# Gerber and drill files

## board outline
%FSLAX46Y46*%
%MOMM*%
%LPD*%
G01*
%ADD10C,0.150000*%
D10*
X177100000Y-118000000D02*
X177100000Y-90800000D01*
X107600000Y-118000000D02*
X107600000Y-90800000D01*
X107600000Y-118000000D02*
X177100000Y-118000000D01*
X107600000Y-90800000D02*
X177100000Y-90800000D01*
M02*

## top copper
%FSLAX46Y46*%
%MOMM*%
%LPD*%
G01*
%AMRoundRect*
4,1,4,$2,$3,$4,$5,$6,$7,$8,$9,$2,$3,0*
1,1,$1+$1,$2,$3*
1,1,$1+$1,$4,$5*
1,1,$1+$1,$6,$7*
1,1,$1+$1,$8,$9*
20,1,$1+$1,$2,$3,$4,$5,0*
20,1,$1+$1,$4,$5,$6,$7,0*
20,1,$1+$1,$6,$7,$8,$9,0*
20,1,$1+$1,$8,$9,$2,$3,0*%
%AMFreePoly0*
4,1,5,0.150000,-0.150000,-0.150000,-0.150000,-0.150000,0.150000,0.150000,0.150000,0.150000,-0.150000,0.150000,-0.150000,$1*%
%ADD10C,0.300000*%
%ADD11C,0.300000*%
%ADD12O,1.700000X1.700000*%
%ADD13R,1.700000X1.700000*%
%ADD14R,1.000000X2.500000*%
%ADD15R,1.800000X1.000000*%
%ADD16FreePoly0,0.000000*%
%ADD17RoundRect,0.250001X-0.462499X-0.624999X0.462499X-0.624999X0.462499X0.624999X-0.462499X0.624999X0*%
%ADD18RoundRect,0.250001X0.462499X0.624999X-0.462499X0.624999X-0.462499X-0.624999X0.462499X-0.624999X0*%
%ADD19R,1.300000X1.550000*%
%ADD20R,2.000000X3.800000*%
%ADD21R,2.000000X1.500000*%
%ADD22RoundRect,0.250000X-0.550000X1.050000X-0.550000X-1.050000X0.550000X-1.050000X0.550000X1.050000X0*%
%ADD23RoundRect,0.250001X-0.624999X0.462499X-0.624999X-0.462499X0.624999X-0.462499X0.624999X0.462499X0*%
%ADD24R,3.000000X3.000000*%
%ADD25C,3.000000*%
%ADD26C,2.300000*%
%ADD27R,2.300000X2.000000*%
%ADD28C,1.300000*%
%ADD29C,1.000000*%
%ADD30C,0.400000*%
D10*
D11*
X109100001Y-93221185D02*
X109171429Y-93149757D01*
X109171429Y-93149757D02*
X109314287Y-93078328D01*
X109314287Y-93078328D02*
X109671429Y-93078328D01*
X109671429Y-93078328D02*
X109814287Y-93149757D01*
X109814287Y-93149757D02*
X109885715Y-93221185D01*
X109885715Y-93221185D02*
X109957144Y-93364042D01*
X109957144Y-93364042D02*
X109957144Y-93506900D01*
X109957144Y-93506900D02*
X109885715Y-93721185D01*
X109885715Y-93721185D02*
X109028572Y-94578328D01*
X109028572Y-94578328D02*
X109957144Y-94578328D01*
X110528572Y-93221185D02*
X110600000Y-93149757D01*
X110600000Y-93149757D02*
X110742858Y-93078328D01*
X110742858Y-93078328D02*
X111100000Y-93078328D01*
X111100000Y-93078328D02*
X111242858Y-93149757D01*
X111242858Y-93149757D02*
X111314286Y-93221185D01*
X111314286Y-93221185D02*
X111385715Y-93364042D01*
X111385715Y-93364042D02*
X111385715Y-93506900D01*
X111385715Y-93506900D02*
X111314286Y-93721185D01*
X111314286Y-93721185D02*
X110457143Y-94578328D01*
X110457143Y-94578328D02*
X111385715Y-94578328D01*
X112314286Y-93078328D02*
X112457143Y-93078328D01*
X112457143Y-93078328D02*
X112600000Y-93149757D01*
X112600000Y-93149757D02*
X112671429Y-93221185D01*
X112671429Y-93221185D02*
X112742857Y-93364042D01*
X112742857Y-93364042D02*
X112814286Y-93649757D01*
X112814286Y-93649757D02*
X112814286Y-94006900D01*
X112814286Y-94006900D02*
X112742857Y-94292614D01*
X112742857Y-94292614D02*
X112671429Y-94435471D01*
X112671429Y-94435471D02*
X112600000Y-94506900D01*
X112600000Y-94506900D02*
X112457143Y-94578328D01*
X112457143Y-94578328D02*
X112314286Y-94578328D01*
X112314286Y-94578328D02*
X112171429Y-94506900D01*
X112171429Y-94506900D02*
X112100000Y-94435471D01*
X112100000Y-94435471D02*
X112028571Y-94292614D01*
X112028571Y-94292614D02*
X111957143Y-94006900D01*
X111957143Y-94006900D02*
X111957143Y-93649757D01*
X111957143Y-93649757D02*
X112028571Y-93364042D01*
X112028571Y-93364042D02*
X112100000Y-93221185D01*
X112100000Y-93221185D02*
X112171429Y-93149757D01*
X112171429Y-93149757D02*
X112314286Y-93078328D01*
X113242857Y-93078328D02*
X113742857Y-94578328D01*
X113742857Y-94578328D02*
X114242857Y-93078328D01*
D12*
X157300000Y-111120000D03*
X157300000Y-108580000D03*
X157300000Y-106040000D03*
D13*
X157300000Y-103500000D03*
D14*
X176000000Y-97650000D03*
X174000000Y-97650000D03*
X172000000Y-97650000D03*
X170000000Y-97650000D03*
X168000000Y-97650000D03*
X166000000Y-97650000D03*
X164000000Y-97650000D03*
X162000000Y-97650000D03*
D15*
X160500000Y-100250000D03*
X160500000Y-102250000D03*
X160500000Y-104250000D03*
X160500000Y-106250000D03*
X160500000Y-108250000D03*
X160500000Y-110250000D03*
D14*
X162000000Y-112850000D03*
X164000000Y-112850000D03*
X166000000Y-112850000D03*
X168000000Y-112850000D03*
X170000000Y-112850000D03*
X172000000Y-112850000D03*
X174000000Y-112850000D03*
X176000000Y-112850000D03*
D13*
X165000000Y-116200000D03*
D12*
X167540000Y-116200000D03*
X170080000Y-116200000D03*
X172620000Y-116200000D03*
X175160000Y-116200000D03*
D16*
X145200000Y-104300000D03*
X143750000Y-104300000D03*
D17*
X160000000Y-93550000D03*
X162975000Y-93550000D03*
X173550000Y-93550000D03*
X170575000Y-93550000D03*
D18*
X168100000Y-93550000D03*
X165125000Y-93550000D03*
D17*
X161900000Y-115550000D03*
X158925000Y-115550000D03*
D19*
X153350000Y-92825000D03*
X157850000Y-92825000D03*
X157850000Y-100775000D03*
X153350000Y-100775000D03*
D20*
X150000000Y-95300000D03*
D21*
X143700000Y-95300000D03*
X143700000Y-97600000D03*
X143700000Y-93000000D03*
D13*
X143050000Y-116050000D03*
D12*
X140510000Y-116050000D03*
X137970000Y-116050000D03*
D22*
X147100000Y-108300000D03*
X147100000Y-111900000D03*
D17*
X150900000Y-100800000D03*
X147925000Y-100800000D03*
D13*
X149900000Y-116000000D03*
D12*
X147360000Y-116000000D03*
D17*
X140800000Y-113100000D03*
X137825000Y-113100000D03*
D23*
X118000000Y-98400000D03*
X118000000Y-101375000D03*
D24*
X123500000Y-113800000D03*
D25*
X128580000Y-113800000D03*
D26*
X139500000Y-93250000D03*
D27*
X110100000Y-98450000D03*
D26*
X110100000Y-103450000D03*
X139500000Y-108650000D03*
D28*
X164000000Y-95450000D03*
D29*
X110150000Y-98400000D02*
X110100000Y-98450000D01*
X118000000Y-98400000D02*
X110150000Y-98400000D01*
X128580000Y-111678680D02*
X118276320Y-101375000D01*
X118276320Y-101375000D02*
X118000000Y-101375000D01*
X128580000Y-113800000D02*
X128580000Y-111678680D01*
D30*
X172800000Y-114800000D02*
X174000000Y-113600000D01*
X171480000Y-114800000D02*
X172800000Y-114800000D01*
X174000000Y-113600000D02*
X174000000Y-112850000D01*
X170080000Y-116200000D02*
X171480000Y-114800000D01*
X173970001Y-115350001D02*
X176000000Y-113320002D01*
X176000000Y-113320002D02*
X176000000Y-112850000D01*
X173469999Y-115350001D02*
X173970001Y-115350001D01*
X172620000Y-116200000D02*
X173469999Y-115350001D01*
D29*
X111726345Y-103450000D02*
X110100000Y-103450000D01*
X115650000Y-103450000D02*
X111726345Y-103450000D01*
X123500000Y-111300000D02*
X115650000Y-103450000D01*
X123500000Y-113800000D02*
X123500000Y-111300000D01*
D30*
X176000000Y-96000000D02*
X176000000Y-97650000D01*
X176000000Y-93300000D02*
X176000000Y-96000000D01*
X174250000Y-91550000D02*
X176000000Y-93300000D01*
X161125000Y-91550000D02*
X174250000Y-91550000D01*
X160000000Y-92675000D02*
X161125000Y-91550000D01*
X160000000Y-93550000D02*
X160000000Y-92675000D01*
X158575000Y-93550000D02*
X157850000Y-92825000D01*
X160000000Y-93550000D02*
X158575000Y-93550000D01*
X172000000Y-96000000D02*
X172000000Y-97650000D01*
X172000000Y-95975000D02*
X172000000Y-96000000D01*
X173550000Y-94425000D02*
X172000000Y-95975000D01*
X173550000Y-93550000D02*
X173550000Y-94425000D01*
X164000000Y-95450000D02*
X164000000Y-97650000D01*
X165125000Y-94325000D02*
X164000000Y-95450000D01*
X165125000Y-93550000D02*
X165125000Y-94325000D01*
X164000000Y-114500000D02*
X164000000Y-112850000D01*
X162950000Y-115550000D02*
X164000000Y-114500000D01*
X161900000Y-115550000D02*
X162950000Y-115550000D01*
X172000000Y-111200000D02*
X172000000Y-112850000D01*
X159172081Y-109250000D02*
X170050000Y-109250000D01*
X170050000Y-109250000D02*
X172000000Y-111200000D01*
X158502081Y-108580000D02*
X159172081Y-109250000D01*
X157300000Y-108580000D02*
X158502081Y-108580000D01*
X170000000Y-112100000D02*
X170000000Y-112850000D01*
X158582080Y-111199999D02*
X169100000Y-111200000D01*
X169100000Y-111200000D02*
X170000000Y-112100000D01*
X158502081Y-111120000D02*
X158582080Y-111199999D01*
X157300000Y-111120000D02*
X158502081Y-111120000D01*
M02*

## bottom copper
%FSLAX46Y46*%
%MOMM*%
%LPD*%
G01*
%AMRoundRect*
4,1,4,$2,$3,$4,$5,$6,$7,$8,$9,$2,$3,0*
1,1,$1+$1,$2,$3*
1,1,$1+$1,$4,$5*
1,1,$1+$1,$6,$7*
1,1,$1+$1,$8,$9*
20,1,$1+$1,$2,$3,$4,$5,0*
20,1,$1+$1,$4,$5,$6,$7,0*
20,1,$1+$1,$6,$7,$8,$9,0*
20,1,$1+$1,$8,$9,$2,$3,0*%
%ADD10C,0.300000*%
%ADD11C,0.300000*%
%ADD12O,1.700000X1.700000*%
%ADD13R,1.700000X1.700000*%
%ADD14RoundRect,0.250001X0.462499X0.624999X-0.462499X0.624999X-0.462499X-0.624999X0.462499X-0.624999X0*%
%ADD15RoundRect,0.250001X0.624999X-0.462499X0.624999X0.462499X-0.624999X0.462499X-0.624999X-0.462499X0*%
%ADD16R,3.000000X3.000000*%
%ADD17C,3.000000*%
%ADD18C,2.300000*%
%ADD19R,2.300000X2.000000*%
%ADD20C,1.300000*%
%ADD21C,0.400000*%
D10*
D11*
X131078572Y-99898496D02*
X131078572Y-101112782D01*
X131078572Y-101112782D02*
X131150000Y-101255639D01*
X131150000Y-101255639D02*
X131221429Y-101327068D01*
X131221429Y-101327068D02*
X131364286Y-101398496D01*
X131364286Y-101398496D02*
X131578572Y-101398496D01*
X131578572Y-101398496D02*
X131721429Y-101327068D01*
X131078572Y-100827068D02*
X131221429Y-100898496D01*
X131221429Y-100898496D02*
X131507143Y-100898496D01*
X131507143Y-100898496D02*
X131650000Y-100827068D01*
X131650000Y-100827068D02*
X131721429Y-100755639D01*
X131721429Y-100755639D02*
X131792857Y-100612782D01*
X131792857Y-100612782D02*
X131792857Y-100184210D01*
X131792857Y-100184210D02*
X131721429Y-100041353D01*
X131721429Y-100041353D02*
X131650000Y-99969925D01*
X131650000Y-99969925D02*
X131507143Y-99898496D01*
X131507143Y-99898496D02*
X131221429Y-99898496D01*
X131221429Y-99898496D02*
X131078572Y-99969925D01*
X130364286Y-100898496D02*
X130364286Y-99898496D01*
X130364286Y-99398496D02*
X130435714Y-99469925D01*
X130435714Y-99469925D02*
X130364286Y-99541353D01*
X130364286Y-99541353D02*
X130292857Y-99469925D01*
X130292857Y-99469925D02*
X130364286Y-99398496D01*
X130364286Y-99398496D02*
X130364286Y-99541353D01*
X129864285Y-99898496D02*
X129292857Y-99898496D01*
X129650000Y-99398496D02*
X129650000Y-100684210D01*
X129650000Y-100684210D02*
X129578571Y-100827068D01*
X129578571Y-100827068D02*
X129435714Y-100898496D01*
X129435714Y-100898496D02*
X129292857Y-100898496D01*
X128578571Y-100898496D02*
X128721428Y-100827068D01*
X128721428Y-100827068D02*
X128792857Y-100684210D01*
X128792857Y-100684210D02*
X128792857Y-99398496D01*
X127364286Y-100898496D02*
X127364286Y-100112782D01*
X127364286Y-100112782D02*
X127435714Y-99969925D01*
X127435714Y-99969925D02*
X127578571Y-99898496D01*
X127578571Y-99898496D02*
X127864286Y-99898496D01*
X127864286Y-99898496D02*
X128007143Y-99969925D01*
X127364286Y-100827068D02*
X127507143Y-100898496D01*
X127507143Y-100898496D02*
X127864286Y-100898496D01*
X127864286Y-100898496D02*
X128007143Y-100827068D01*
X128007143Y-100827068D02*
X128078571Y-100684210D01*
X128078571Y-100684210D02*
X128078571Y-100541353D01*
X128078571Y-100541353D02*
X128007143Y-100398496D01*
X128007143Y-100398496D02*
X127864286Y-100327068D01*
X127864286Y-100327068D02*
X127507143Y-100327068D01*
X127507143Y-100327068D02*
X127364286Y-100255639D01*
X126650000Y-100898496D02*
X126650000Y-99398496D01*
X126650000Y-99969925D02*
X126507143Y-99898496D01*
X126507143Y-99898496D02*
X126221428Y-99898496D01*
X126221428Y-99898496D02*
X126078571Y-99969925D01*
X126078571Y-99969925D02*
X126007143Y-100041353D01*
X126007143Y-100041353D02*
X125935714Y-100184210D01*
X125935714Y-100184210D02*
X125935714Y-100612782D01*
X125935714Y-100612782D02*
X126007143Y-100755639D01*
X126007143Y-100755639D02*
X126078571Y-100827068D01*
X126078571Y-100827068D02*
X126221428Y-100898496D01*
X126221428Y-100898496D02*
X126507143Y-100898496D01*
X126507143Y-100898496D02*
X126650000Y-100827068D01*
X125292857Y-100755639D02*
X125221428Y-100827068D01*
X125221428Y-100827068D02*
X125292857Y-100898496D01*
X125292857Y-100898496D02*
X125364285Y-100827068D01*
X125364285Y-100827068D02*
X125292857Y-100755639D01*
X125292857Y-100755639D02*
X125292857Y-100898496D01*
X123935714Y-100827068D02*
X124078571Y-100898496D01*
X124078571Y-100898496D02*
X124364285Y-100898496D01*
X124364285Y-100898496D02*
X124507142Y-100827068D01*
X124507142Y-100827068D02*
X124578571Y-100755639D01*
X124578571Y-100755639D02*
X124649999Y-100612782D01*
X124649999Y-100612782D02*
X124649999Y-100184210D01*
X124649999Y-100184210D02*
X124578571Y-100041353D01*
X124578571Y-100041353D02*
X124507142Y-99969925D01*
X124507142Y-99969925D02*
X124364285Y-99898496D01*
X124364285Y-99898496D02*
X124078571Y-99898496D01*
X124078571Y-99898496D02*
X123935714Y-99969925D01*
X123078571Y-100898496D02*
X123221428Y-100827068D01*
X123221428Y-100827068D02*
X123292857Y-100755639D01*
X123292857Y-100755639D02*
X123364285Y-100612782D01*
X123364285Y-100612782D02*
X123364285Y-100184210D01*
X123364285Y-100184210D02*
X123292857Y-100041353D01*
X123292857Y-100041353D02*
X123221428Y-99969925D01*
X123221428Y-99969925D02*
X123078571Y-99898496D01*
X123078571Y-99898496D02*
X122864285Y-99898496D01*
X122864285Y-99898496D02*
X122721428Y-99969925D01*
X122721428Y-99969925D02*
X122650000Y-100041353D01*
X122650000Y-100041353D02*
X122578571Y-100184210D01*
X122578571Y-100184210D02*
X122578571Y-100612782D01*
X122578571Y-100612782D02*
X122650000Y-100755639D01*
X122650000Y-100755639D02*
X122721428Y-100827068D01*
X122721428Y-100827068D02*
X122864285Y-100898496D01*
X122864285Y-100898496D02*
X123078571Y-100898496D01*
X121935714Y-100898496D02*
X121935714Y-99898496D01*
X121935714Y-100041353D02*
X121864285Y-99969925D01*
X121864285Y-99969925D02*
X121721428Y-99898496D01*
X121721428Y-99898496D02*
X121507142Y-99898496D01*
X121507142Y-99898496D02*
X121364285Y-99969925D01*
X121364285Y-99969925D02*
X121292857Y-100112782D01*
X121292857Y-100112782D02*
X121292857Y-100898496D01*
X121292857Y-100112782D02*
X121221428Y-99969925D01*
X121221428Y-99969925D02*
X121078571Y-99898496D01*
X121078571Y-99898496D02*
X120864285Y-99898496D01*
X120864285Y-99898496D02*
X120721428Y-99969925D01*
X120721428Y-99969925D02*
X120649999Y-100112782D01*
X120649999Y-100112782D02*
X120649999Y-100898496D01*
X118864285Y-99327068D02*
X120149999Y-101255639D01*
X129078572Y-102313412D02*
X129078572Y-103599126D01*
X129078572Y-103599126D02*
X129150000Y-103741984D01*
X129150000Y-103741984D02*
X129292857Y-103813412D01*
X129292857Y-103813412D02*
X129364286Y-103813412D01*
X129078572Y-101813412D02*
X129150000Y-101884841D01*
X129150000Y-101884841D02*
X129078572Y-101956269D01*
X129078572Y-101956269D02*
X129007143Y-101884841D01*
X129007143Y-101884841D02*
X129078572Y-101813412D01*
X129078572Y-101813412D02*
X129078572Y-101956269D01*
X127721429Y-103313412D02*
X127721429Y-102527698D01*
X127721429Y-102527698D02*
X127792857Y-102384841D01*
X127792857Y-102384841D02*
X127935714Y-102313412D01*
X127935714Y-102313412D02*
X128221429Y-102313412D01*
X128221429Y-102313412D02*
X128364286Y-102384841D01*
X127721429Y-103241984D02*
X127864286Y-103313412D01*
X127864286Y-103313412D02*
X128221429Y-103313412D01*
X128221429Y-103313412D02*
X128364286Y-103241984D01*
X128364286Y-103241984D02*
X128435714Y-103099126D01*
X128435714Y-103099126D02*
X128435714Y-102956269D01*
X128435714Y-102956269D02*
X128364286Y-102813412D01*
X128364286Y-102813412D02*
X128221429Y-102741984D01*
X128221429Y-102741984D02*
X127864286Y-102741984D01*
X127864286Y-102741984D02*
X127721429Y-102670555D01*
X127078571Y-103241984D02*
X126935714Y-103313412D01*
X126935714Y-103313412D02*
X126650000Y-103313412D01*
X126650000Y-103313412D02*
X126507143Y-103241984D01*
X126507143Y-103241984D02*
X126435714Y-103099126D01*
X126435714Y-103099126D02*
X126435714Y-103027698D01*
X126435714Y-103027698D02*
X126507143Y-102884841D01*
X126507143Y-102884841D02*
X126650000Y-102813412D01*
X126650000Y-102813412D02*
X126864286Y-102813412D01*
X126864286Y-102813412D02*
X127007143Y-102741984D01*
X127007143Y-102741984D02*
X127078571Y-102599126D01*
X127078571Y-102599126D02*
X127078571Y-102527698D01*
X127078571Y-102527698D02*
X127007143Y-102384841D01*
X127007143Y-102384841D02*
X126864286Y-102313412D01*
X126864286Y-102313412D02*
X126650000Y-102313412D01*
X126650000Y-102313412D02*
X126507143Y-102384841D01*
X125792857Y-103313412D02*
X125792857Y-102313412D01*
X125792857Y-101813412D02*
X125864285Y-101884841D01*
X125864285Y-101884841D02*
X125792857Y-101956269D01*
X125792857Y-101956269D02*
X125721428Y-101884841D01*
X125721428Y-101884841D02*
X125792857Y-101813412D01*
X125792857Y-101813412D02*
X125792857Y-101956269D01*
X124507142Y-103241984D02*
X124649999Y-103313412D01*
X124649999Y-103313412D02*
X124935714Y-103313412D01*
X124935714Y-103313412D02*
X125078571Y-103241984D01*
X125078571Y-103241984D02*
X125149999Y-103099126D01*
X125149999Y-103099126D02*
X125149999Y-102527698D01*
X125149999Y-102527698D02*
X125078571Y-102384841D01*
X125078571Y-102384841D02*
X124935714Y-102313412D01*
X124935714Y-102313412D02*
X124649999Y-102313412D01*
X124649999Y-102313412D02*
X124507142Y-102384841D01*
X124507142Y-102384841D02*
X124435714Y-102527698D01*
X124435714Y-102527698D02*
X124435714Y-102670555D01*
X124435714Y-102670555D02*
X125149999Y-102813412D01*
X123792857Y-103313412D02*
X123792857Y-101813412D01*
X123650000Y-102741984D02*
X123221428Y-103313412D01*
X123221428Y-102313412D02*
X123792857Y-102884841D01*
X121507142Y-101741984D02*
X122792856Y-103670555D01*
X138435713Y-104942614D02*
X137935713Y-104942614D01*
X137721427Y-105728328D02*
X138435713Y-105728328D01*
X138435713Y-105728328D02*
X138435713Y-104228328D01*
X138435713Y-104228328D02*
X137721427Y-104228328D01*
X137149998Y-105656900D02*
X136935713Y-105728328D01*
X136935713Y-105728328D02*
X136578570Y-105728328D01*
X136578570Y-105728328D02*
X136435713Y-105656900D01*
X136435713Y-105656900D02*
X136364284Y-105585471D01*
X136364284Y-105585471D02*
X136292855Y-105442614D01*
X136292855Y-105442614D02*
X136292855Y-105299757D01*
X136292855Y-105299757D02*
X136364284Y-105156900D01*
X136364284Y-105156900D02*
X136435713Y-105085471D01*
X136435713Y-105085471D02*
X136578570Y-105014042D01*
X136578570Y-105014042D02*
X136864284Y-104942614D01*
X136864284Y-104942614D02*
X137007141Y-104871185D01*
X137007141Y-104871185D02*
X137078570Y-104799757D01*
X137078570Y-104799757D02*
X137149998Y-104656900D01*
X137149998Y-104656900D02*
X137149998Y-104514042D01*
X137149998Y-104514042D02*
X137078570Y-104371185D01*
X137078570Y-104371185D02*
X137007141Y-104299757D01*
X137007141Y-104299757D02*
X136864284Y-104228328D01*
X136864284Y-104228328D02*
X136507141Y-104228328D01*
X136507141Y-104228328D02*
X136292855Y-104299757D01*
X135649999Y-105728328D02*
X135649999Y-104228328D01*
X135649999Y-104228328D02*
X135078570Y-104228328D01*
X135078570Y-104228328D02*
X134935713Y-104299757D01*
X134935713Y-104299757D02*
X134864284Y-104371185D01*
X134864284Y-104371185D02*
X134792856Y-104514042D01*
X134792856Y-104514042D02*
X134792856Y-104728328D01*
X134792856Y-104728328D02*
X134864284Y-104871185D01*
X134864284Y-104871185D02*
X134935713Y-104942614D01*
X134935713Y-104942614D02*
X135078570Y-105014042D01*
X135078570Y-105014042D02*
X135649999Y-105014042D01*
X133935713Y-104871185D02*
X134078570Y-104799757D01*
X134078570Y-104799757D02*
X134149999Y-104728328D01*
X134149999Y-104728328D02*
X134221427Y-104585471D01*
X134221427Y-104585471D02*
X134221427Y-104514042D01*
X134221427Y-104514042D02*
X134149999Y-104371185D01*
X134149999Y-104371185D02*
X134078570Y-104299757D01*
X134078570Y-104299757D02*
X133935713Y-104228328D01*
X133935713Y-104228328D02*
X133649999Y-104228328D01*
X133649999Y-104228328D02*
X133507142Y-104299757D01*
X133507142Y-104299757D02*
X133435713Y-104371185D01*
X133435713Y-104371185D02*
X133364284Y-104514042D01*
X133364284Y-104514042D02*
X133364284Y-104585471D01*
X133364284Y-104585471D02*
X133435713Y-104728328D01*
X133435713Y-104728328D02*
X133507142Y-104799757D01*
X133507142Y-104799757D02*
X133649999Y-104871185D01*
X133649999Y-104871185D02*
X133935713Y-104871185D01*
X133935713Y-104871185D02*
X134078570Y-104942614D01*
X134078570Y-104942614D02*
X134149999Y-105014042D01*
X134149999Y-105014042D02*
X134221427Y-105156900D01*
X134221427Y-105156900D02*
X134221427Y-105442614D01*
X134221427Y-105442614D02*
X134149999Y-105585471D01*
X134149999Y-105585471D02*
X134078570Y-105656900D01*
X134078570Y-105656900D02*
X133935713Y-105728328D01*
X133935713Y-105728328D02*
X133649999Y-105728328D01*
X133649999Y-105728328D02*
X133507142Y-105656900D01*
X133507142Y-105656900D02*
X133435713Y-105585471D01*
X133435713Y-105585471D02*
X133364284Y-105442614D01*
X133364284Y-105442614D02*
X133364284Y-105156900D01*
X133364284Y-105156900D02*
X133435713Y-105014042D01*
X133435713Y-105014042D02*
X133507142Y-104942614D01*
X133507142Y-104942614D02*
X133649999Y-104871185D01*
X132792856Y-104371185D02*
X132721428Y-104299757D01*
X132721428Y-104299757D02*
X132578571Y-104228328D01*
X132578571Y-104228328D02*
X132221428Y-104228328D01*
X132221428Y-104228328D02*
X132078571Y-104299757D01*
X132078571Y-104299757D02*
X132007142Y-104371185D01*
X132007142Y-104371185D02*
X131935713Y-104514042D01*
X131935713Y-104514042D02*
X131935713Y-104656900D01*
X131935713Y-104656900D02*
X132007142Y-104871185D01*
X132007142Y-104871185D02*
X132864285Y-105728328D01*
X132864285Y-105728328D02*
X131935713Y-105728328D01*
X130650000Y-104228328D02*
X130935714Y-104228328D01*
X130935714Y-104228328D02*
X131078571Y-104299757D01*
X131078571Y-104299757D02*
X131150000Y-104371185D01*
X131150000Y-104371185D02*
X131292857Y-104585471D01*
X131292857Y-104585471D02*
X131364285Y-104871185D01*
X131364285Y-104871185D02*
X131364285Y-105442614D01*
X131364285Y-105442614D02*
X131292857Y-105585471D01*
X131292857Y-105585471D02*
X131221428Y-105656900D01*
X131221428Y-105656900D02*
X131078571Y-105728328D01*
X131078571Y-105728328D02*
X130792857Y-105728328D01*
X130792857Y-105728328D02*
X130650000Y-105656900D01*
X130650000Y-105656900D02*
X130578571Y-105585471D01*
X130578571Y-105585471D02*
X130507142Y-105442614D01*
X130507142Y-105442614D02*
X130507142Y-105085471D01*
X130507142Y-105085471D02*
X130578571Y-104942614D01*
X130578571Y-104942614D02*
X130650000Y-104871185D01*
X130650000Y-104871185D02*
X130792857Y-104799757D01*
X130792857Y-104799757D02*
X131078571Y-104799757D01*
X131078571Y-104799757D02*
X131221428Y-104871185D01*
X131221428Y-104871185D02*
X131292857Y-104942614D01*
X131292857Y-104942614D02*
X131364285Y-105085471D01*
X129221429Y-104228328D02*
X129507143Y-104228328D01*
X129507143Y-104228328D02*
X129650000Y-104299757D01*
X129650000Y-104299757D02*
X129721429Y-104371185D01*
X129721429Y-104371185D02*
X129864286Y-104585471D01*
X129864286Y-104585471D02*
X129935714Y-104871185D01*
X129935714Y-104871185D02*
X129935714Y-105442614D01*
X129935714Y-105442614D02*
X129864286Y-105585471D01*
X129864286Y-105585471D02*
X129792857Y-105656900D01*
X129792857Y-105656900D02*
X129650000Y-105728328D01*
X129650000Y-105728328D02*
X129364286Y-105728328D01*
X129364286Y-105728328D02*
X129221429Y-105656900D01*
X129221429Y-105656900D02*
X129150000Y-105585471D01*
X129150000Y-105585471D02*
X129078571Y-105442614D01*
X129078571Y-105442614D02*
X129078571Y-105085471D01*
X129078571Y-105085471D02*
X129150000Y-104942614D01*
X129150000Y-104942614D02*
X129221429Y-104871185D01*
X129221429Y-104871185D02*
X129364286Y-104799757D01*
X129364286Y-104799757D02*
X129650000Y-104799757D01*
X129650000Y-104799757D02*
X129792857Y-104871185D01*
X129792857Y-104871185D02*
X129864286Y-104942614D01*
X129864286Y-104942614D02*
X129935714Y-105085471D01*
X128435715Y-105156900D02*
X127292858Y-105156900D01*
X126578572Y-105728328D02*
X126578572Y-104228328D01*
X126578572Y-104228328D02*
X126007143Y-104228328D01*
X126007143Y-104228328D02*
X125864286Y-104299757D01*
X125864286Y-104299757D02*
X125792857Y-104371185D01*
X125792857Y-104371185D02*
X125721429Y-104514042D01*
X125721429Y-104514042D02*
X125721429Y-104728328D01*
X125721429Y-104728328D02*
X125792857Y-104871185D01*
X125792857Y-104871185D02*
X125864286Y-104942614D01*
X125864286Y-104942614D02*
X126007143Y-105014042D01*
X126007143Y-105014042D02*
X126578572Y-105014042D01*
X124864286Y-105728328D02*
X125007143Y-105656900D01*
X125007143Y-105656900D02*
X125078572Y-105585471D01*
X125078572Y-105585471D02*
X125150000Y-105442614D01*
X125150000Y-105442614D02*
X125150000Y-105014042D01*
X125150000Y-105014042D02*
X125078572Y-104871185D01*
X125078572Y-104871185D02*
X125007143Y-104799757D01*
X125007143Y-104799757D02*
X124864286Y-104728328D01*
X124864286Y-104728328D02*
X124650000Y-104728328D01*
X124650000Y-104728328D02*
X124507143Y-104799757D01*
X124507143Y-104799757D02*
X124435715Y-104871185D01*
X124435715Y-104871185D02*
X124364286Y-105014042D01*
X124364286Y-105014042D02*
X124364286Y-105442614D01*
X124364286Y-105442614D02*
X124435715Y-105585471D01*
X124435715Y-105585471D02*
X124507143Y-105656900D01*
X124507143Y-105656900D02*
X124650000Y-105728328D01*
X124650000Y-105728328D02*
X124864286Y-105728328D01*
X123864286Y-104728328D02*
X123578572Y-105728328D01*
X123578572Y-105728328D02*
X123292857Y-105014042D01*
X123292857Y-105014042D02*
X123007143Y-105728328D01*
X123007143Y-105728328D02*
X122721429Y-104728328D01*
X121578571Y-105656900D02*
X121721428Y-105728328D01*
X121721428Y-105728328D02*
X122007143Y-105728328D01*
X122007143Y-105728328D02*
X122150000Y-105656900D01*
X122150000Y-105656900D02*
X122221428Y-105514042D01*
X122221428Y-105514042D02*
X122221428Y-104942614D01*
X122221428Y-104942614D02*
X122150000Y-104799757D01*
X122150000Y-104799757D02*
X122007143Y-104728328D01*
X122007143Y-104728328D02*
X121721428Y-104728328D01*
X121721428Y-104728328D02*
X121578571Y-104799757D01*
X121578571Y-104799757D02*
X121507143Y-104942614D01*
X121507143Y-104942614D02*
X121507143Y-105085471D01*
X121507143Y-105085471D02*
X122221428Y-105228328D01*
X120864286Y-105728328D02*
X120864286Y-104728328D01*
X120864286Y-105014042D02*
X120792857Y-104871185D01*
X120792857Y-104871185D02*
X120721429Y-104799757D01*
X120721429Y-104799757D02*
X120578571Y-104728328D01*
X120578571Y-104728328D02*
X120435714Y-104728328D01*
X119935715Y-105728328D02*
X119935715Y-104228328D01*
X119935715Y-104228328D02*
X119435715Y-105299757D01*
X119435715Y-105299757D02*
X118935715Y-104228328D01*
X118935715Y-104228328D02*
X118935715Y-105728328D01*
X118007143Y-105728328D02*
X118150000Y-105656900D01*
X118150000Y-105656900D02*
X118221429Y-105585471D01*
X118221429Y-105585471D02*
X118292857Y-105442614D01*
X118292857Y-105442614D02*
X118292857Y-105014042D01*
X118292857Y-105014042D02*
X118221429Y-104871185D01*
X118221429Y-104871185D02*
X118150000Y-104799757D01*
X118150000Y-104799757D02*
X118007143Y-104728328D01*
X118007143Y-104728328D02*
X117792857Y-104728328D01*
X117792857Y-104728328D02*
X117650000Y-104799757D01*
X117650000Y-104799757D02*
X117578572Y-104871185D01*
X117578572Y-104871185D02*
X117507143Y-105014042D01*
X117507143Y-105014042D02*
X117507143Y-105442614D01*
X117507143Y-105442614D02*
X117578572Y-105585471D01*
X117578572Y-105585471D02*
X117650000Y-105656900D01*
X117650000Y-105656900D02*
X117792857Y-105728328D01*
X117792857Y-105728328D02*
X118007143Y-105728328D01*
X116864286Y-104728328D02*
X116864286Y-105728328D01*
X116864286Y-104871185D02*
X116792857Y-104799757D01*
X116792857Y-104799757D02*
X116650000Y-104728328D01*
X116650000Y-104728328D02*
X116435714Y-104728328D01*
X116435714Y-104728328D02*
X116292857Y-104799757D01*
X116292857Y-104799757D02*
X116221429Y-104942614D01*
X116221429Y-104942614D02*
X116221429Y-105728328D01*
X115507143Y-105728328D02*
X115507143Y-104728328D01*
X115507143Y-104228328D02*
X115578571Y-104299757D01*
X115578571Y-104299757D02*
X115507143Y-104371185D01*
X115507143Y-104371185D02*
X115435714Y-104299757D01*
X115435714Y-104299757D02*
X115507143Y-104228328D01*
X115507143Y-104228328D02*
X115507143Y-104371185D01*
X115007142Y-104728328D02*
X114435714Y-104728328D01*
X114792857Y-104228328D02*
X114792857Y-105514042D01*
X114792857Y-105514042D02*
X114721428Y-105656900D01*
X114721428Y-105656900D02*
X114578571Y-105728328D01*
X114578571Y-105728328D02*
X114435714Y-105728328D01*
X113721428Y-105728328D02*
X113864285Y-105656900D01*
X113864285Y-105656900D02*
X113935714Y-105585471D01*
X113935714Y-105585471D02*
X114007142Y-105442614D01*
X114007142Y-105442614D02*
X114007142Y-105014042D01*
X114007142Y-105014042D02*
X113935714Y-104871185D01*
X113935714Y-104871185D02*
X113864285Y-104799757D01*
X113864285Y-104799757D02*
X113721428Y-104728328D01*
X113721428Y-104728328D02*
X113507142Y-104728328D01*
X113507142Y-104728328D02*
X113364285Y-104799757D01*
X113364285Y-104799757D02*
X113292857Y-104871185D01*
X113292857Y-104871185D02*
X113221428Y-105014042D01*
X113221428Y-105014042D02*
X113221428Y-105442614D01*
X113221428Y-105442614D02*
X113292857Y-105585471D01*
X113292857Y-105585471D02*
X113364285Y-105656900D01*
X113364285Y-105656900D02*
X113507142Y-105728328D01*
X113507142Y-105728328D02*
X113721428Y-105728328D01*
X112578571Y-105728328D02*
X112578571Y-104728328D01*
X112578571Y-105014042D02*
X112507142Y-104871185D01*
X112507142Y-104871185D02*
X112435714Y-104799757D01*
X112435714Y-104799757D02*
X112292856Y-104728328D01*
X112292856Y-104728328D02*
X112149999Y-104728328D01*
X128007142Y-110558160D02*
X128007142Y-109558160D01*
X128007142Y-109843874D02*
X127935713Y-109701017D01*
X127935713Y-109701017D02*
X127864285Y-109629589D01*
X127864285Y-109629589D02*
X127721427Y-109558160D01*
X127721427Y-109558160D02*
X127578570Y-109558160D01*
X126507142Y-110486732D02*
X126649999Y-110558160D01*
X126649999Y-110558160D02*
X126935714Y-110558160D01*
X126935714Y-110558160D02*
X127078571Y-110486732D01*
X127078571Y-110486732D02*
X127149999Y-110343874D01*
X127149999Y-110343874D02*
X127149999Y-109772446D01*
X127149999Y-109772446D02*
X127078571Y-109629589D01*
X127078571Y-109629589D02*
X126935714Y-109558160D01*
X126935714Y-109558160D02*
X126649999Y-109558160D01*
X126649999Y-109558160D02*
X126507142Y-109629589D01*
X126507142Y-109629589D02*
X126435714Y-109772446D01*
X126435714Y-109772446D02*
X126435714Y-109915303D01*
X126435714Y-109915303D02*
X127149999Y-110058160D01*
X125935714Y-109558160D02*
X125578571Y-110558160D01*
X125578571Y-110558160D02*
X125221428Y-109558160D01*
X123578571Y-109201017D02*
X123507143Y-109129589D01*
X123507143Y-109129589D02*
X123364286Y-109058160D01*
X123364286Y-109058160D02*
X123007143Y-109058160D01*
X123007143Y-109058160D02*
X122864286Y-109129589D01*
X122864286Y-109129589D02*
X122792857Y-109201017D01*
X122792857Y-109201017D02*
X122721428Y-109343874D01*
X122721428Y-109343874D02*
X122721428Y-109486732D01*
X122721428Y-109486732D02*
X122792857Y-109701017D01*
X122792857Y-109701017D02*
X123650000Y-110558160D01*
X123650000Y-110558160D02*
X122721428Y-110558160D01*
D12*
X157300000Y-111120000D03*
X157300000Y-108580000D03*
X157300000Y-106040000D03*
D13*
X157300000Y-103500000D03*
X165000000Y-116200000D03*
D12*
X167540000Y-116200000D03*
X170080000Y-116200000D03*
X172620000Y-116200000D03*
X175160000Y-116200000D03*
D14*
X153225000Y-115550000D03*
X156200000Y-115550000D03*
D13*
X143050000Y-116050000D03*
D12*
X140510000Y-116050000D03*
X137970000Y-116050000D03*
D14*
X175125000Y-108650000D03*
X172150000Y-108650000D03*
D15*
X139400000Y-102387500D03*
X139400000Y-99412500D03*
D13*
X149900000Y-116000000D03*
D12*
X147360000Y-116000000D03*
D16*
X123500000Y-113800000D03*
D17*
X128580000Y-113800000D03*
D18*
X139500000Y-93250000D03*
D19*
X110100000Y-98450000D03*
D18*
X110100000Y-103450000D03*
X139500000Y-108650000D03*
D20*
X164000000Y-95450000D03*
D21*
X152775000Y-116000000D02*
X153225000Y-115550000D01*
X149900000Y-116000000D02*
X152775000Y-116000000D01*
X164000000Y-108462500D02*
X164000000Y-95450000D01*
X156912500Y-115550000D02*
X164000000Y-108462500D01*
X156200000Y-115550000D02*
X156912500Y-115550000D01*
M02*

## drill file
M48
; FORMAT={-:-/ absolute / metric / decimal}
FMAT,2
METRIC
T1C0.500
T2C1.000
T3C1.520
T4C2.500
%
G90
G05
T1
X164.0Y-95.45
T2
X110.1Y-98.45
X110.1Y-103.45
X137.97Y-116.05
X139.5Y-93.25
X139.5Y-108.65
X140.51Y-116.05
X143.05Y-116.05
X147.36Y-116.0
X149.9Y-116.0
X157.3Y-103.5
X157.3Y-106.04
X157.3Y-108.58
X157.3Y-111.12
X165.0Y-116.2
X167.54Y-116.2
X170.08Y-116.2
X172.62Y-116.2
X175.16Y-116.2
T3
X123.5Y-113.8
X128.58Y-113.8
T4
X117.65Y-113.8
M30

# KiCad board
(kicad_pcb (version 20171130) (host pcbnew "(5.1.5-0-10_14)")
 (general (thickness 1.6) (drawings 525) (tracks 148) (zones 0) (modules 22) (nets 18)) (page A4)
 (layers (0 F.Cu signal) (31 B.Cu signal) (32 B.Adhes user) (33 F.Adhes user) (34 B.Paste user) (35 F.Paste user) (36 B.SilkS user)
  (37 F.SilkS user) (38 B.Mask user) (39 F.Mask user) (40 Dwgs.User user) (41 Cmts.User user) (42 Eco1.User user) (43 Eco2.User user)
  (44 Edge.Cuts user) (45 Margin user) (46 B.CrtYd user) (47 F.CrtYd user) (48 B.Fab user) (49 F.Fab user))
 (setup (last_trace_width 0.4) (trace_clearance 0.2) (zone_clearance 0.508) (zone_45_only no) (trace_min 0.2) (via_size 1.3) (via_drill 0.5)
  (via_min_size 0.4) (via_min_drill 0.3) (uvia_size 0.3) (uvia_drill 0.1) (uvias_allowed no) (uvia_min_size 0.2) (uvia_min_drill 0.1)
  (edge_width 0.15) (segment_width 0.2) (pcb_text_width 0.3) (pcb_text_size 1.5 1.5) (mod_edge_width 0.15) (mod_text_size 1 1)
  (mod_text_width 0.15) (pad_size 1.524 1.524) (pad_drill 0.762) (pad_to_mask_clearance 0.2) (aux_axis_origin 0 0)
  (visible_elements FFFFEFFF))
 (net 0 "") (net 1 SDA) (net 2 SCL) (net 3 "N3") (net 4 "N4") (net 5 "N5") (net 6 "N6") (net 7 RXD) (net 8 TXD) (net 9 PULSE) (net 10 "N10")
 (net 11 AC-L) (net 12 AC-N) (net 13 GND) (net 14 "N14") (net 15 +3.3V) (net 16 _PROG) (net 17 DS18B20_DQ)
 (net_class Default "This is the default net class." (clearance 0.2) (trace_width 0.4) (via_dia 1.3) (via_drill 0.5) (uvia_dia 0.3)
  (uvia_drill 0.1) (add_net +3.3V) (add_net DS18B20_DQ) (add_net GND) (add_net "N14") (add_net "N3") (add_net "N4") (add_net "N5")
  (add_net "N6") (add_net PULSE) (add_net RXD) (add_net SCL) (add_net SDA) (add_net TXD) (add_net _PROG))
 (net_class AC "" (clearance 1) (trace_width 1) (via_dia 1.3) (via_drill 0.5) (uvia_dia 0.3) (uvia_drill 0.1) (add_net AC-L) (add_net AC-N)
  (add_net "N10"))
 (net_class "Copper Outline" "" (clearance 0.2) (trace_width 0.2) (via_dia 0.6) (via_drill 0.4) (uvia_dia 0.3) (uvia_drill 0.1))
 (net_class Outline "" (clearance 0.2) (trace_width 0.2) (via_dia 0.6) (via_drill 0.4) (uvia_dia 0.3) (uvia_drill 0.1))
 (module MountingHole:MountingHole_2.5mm (layer F.Cu) (at 117.65 113.8)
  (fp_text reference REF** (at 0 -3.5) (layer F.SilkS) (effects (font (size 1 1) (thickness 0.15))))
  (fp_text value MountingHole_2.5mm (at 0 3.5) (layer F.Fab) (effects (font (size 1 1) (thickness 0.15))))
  (pad 1 np_thru_hole circle (at 0 0) (size 2.5 2.5) (drill 2.5) (layers *.Cu *.Mask)))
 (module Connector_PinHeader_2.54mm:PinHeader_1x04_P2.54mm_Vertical (layer F.Cu) (at 157.3 103.5)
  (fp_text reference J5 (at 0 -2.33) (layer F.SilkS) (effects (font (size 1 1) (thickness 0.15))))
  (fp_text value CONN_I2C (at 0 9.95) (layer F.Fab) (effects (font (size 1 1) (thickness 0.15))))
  (pad 4 thru_hole oval (at 0 7.62) (size 1.7 1.7) (drill 1) (layers *.Cu *.Mask) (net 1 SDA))
  (pad 3 thru_hole oval (at 0 5.08) (size 1.7 1.7) (drill 1) (layers *.Cu *.Mask) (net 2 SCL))
  (pad 2 thru_hole oval (at 0 2.54) (size 1.7 1.7) (drill 1) (layers *.Cu *.Mask))
  (pad 1 thru_hole rect (at 0 0) (size 1.7 1.7) (drill 1) (layers *.Cu *.Mask)))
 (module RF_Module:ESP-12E (layer F.Cu) (at 172.5 105.25 270)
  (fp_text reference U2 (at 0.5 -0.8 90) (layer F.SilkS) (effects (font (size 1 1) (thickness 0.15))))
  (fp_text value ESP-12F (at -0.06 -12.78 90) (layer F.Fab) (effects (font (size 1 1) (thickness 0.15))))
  (pad 1 smd rect (at -7.6 -3.5 270) (size 2.5 1) (layers F.Cu F.Paste F.Mask) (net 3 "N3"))
  (pad 2 smd rect (at -7.6 -1.5 270) (size 2.5 1) (layers F.Cu F.Paste F.Mask))
  (pad 3 smd rect (at -7.6 0.5 270) (size 2.5 1) (layers F.Cu F.Paste F.Mask) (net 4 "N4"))
  (pad 4 smd rect (at -7.6 2.5 270) (size 2.5 1) (layers F.Cu F.Paste F.Mask))
  (pad 5 smd rect (at -7.6 4.5 270) (size 2.5 1) (layers F.Cu F.Paste F.Mask))
  (pad 6 smd rect (at -7.6 6.5 270) (size 2.5 1) (layers F.Cu F.Paste F.Mask))
  (pad 7 smd rect (at -7.6 8.5 270) (size 2.5 1) (layers F.Cu F.Paste F.Mask) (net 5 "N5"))
  (pad 8 smd rect (at -7.6 10.5 270) (size 2.5 1) (layers F.Cu F.Paste F.Mask))
  (pad 9 smd rect (at -5 12 270) (size 1 1.8) (layers F.Cu F.Paste F.Mask))
  (pad 10 smd rect (at -3 12 270) (size 1 1.8) (layers F.Cu F.Paste F.Mask))
  (pad 11 smd rect (at -1 12 270) (size 1 1.8) (layers F.Cu F.Paste F.Mask))
  (pad 12 smd rect (at 1 12 270) (size 1 1.8) (layers F.Cu F.Paste F.Mask))
  (pad 13 smd rect (at 3 12 270) (size 1 1.8) (layers F.Cu F.Paste F.Mask))
  (pad 14 smd rect (at 5 12 270) (size 1 1.8) (layers F.Cu F.Paste F.Mask))
  (pad 15 smd rect (at 7.6 10.5 270) (size 2.5 1) (layers F.Cu F.Paste F.Mask))
  (pad 16 smd rect (at 7.6 8.5 270) (size 2.5 1) (layers F.Cu F.Paste F.Mask) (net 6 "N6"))
  (pad 17 smd rect (at 7.6 6.5 270) (size 2.5 1) (layers F.Cu F.Paste F.Mask))
  (pad 18 smd rect (at 7.6 4.5 270) (size 2.5 1) (layers F.Cu F.Paste F.Mask))
  (pad 19 smd rect (at 7.6 2.5 270) (size 2.5 1) (layers F.Cu F.Paste F.Mask) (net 1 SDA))
  (pad 20 smd rect (at 7.6 0.5 270) (size 2.5 1) (layers F.Cu F.Paste F.Mask) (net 2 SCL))
  (pad 21 smd rect (at 7.6 -1.5 270) (size 2.5 1) (layers F.Cu F.Paste F.Mask) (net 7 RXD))
  (pad 22 smd rect (at 7.6 -3.5 270) (size 2.5 1) (layers F.Cu F.Paste F.Mask) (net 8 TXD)))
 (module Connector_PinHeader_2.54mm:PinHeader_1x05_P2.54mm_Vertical (layer F.Cu) (at 165 116.2 90)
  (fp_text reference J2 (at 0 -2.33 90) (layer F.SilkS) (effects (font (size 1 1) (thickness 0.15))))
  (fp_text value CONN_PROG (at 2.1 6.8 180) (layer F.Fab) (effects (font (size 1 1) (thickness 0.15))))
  (pad 1 thru_hole rect (at 0 0 90) (size 1.7 1.7) (drill 1) (layers *.Cu *.Mask))
  (pad 2 thru_hole oval (at 0 2.54 90) (size 1.7 1.7) (drill 1) (layers *.Cu *.Mask))
  (pad 3 thru_hole oval (at 0 5.08 90) (size 1.7 1.7) (drill 1) (layers *.Cu *.Mask) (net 7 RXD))
  (pad 4 thru_hole oval (at 0 7.62 90) (size 1.7 1.7) (drill 1) (layers *.Cu *.Mask) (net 8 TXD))
  (pad 5 thru_hole oval (at 0 10.16 90) (size 1.7 1.7) (drill 1) (layers *.Cu *.Mask)))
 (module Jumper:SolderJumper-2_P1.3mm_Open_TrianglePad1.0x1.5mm (layer F.Cu) (at 144.475 104.3)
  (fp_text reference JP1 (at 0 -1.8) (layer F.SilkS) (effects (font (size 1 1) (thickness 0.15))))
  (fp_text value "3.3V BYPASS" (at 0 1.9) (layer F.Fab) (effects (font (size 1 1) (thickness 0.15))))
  (pad 2 smd custom (at 0.725 0) (size 0.3 0.3) (layers F.Cu F.Mask) (zone_connect 2) (options (clearance outline) (anchor rect))
   (primitives))
  (pad 1 smd custom (at -0.725 0) (size 0.3 0.3) (layers F.Cu F.Mask) (zone_connect 2) (options (clearance outline) (anchor rect))
   (primitives)))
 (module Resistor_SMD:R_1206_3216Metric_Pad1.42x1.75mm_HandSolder (layer F.Cu) (at 161.4875 93.55)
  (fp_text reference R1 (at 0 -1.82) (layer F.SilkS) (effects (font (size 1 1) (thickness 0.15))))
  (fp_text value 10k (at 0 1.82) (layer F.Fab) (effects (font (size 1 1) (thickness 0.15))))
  (pad 1 smd roundrect (at -1.4875 0) (size 1.425 1.75) (layers F.Cu F.Paste F.Mask) (roundrect_rratio 0.175439) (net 3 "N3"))
  (pad 2 smd roundrect (at 1.4875 0) (size 1.425 1.75) (layers F.Cu F.Paste F.Mask) (roundrect_rratio 0.175439)))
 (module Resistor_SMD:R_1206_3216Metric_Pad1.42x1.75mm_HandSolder (layer F.Cu) (at 172.0625 93.55)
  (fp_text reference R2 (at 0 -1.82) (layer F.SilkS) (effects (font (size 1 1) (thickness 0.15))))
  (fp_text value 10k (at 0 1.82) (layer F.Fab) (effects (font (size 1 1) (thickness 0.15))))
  (pad 2 smd roundrect (at 1.4875 0) (size 1.425 1.75) (layers F.Cu F.Paste F.Mask) (roundrect_rratio 0.175439) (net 4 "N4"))
  (pad 1 smd roundrect (at -1.4875 0) (size 1.425 1.75) (layers F.Cu F.Paste F.Mask) (roundrect_rratio 0.175439)))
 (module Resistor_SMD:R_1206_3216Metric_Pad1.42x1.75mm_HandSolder (layer B.Cu) (at 154.7125 115.55 180)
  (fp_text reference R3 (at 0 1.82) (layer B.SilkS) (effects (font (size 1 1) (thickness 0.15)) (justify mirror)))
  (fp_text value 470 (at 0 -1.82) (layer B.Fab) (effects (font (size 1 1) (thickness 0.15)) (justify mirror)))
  (pad 2 smd roundrect (at 1.4875 0 180) (size 1.425 1.75) (layers B.Cu B.Paste B.Mask) (roundrect_rratio 0.175439) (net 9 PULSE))
  (pad 1 smd roundrect (at -1.4875 0 180) (size 1.425 1.75) (layers B.Cu B.Paste B.Mask) (roundrect_rratio 0.175439) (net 5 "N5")))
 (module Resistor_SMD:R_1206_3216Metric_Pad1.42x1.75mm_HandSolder (layer F.Cu) (at 166.6125 93.55 180)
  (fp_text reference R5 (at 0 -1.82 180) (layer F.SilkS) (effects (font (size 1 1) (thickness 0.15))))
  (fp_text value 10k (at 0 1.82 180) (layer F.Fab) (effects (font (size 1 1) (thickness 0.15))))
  (pad 1 smd roundrect (at -1.4875 0 180) (size 1.425 1.75) (layers F.Cu F.Paste F.Mask) (roundrect_rratio 0.175439))
  (pad 2 smd roundrect (at 1.4875 0 180) (size 1.425 1.75) (layers F.Cu F.Paste F.Mask) (roundrect_rratio 0.175439) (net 5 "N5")))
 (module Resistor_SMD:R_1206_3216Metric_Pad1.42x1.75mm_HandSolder (layer F.Cu) (at 160.4125 115.55)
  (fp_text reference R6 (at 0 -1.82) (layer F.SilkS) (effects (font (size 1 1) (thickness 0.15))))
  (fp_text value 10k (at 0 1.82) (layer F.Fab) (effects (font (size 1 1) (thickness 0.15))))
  (pad 2 smd roundrect (at 1.4875 0) (size 1.425 1.75) (layers F.Cu F.Paste F.Mask) (roundrect_rratio 0.175439) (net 6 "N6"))
  (pad 1 smd roundrect (at -1.4875 0) (size 1.425 1.75) (layers F.Cu F.Paste F.Mask) (roundrect_rratio 0.175439)))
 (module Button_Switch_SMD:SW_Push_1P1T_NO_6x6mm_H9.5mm (layer F.Cu) (at 155.6 96.8 270)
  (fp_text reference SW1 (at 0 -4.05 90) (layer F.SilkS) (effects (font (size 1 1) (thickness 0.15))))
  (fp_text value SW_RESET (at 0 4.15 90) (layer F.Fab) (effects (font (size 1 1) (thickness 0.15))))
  (pad 2 smd rect (at -3.975 2.25 270) (size 1.55 1.3) (layers F.Cu F.Paste F.Mask))
  (pad 1 smd rect (at -3.975 -2.25 270) (size 1.55 1.3) (layers F.Cu F.Paste F.Mask) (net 3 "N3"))
  (pad 1 smd rect (at 3.975 -2.25 270) (size 1.55 1.3) (layers F.Cu F.Paste F.Mask))
  (pad 2 smd rect (at 3.975 2.25 270) (size 1.55 1.3) (layers F.Cu F.Paste F.Mask)))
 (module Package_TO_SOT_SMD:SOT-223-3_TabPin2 (layer F.Cu) (at 146.85 95.3)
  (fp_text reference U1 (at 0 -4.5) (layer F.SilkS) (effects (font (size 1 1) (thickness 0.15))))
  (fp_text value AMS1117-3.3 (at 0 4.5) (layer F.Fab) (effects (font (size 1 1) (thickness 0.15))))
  (pad 2 smd rect (at 3.15 0) (size 2 3.8) (layers F.Cu F.Paste F.Mask))
  (pad 2 smd rect (at -3.15 0) (size 2 1.5) (layers F.Cu F.Paste F.Mask))
  (pad 3 smd rect (at -3.15 2.3) (size 2 1.5) (layers F.Cu F.Paste F.Mask))
  (pad 1 smd rect (at -3.15 -2.3) (size 2 1.5) (layers F.Cu F.Paste F.Mask)))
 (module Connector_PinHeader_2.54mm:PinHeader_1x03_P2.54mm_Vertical (layer F.Cu) (at 143.05 116.05 270)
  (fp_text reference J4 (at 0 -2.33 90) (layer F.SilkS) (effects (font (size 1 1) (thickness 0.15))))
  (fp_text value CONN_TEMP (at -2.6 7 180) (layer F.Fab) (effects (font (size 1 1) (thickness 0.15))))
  (pad 1 thru_hole rect (at 0 0 270) (size 1.7 1.7) (drill 1) (layers *.Cu *.Mask))
  (pad 2 thru_hole oval (at 0 2.54 270) (size 1.7 1.7) (drill 1) (layers *.Cu *.Mask))
  (pad 3 thru_hole oval (at 0 5.08 270) (size 1.7 1.7) (drill 1) (layers *.Cu *.Mask)))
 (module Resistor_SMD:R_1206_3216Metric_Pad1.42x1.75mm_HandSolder (layer B.Cu) (at 173.6375 108.65 180)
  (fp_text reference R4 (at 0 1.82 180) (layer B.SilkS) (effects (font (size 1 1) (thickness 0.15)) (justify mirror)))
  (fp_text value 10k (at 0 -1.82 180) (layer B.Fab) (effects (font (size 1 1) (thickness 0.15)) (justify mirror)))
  (pad 1 smd roundrect (at -1.4875 0 180) (size 1.425 1.75) (layers B.Cu B.Paste B.Mask) (roundrect_rratio 0.175439))
  (pad 2 smd roundrect (at 1.4875 0 180) (size 1.425 1.75) (layers B.Cu B.Paste B.Mask) (roundrect_rratio 0.175439)))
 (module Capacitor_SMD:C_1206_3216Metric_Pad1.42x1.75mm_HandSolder (layer B.Cu) (at 139.4 100.9 90)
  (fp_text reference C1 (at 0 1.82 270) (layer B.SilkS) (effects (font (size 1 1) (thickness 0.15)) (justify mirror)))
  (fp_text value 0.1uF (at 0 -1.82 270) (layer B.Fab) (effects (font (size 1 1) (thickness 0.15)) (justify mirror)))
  (pad 1 smd roundrect (at -1.4875 0 90) (size 1.425 1.75) (layers B.Cu B.Paste B.Mask) (roundrect_rratio 0.175439))
  (pad 2 smd roundrect (at 1.4875 0 90) (size 1.425 1.75) (layers B.Cu B.Paste B.Mask) (roundrect_rratio 0.175439)))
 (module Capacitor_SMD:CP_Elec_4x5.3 (layer F.Cu) (at 147.1 110.1 270)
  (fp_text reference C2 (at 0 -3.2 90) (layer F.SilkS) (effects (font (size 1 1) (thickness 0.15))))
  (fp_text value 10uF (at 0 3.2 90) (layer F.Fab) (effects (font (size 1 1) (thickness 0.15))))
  (pad 1 smd roundrect (at -1.8 0 270) (size 2.6 1.6) (layers F.Cu F.Paste F.Mask) (roundrect_rratio 0.15625))
  (pad 2 smd roundrect (at 1.8 0 270) (size 2.6 1.6) (layers F.Cu F.Paste F.Mask) (roundrect_rratio 0.15625)))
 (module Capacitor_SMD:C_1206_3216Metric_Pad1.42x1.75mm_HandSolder (layer F.Cu) (at 149.4125 100.8)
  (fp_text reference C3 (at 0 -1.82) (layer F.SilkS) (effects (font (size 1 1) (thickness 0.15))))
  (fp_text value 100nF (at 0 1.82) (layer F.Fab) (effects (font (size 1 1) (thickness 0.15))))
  (pad 2 smd roundrect (at 1.4875 0) (size 1.425 1.75) (layers F.Cu F.Paste F.Mask) (roundrect_rratio 0.175439))
  (pad 1 smd roundrect (at -1.4875 0) (size 1.425 1.75) (layers F.Cu F.Paste F.Mask) (roundrect_rratio 0.175439)))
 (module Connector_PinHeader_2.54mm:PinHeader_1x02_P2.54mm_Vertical (layer F.Cu) (at 149.9 116 270)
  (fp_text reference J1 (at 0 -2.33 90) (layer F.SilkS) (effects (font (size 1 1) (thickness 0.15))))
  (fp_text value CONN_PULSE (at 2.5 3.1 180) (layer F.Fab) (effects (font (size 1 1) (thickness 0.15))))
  (pad 1 thru_hole rect (at 0 0 270) (size 1.7 1.7) (drill 1) (layers *.Cu *.Mask) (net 9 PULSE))
  (pad 2 thru_hole oval (at 0 2.54 270) (size 1.7 1.7) (drill 1) (layers *.Cu *.Mask)))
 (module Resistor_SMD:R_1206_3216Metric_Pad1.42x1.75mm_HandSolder (layer F.Cu) (at 139.3125 113.1)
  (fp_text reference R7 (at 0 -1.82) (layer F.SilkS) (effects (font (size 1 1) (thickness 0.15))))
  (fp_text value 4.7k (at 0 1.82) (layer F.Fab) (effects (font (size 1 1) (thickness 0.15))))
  (pad 2 smd roundrect (at 1.4875 0) (size 1.425 1.75) (layers F.Cu F.Paste F.Mask) (roundrect_rratio 0.175439))
  (pad 1 smd roundrect (at -1.4875 0) (size 1.425 1.75) (layers F.Cu F.Paste F.Mask) (roundrect_rratio 0.175439)))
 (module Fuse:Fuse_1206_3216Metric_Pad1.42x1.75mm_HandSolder (layer F.Cu) (at 118 99.8875 270)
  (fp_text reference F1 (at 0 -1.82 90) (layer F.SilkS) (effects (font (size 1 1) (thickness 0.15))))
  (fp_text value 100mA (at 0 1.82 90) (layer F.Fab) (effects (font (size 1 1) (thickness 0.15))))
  (pad 1 smd roundrect (at -1.4875 0 270) (size 1.425 1.75) (layers F.Cu F.Paste F.Mask) (roundrect_rratio 0.175439) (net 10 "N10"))
  (pad 2 smd roundrect (at 1.4875 0 270) (size 1.425 1.75) (layers F.Cu F.Paste F.Mask) (roundrect_rratio 0.175439) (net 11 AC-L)))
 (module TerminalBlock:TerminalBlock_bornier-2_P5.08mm (layer F.Cu) (at 123.5 113.8)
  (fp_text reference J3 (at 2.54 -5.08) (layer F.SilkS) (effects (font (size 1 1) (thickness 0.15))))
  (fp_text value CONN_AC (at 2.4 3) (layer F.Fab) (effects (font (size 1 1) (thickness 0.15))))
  (pad 1 thru_hole rect (at 0 0) (size 3 3) (drill 1.52) (layers *.Cu *.Mask) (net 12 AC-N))
  (pad 2 thru_hole circle (at 5.08 0) (size 3 3) (drill 1.52) (layers *.Cu *.Mask) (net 11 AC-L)))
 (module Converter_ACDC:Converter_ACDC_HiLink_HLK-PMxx (layer F.Cu) (at 110.1 98.45)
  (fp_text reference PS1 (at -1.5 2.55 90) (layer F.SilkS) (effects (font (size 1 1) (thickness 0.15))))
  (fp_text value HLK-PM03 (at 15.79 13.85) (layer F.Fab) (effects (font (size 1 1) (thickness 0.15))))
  (pad 3 thru_hole circle (at 29.4 -5.2) (size 2.3 2.3) (drill 1) (layers *.Cu *.Mask))
  (pad 1 thru_hole rect (at 0 0) (size 2.3 2) (drill 1) (layers *.Cu *.Mask) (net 10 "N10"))
  (pad 2 thru_hole circle (at 0 5) (size 2.3 2.3) (drill 1) (layers *.Cu *.Mask) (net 12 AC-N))
  (pad 4 thru_hole circle (at 29.4 10.2) (size 2.3 2.3) (drill 1) (layers *.Cu *.Mask)))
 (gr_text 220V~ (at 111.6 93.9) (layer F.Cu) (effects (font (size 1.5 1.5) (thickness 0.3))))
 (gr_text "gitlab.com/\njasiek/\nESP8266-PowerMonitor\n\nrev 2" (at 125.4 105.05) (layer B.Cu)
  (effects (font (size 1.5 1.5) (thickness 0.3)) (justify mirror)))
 (gr_line (start 177.1 118) (end 177.1 90.8) (layer Edge.Cuts) (width 0.15))
 (gr_line (start 107.6 118) (end 107.6 90.8) (layer Edge.Cuts) (width 0.15))
 (gr_line (start 107.6 118) (end 177.1 118) (layer Edge.Cuts) (width 0.15))
 (gr_line (start 107.6 90.8) (end 177.1 90.8) (layer Edge.Cuts) (width 0.15))
 (segment (start 110.15 98.4) (end 110.1 98.45) (width 1) (layer F.Cu) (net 10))
 (segment (start 118 98.4) (end 110.15 98.4) (width 1) (layer F.Cu) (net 10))
 (segment (start 128.58 111.67868) (end 118.27632 101.375) (width 1) (layer F.Cu) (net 11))
 (segment (start 118.27632 101.375) (end 118 101.375) (width 1) (layer F.Cu) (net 11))
 (segment (start 128.58 113.8) (end 128.58 111.67868) (width 1) (layer F.Cu) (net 11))
 (segment (start 152.775 116) (end 153.225 115.55) (width 0.4) (layer B.Cu) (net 9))
 (segment (start 149.9 116) (end 152.775 116) (width 0.4) (layer B.Cu) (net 9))
 (segment (start 172.8 114.8) (end 174 113.6) (width 0.4) (layer F.Cu) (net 7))
 (segment (start 171.48 114.8) (end 172.8 114.8) (width 0.4) (layer F.Cu) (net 7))
 (segment (start 174 113.6) (end 174 112.85) (width 0.4) (layer F.Cu) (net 7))
 (segment (start 170.08 116.2) (end 171.48 114.8) (width 0.4) (layer F.Cu) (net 7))
 (segment (start 173.970001 115.350001) (end 176 113.320002) (width 0.4) (layer F.Cu) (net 8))
 (segment (start 176 113.320002) (end 176 112.85) (width 0.4) (layer F.Cu) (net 8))
 (segment (start 173.469999 115.350001) (end 173.970001 115.350001) (width 0.4) (layer F.Cu) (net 8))
 (segment (start 172.62 116.2) (end 173.469999 115.350001) (width 0.4) (layer F.Cu) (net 8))
 (segment (start 111.726345 103.45) (end 110.1 103.45) (width 1) (layer F.Cu) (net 12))
 (segment (start 115.65 103.45) (end 111.726345 103.45) (width 1) (layer F.Cu) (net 12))
 (segment (start 123.5 111.3) (end 115.65 103.45) (width 1) (layer F.Cu) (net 12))
 (segment (start 123.5 113.8) (end 123.5 111.3) (width 1) (layer F.Cu) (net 12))
 (segment (start 176 96) (end 176 97.65) (width 0.4) (layer F.Cu) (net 3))
 (segment (start 176 93.3) (end 176 96) (width 0.4) (layer F.Cu) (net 3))
 (segment (start 174.25 91.55) (end 176 93.3) (width 0.4) (layer F.Cu) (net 3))
 (segment (start 161.125 91.55) (end 174.25 91.55) (width 0.4) (layer F.Cu) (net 3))
 (segment (start 160 92.675) (end 161.125 91.55) (width 0.4) (layer F.Cu) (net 3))
 (segment (start 160 93.55) (end 160 92.675) (width 0.4) (layer F.Cu) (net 3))
 (segment (start 158.575 93.55) (end 157.85 92.825) (width 0.4) (layer F.Cu) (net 3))
 (segment (start 160 93.55) (end 158.575 93.55) (width 0.4) (layer F.Cu) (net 3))
 (segment (start 172 96) (end 172 97.65) (width 0.4) (layer F.Cu) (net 4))
 (segment (start 172 95.975) (end 172 96) (width 0.4) (layer F.Cu) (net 4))
 (segment (start 173.55 94.425) (end 172 95.975) (width 0.4) (layer F.Cu) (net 4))
 (segment (start 173.55 93.55) (end 173.55 94.425) (width 0.4) (layer F.Cu) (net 4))
 (segment (start 164 108.4625) (end 164 95.45) (width 0.4) (layer B.Cu) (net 5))
 (segment (start 156.9125 115.55) (end 164 108.4625) (width 0.4) (layer B.Cu) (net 5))
 (segment (start 156.2 115.55) (end 156.9125 115.55) (width 0.4) (layer B.Cu) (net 5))
 (segment (start 164 95.45) (end 164 97.65) (width 0.4) (layer F.Cu) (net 5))
 (segment (start 165.125 94.325) (end 164 95.45) (width 0.4) (layer F.Cu) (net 5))
 (segment (start 165.125 93.55) (end 165.125 94.325) (width 0.4) (layer F.Cu) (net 5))
 (segment (start 164 114.5) (end 164 112.85) (width 0.4) (layer F.Cu) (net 6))
 (segment (start 162.95 115.55) (end 164 114.5) (width 0.4) (layer F.Cu) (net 6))
 (segment (start 161.9 115.55) (end 162.95 115.55) (width 0.4) (layer F.Cu) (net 6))
 (segment (start 172 111.2) (end 172 112.85) (width 0.4) (layer F.Cu) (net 2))
 (segment (start 159.172081 109.25) (end 170.05 109.25) (width 0.4) (layer F.Cu) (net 2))
 (segment (start 170.05 109.25) (end 172 111.2) (width 0.4) (layer F.Cu) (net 2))
 (segment (start 158.502081 108.58) (end 159.172081 109.25) (width 0.4) (layer F.Cu) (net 2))
 (segment (start 157.3 108.58) (end 158.502081 108.58) (width 0.4) (layer F.Cu) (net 2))
 (segment (start 170 112.1) (end 170 112.85) (width 0.4) (layer F.Cu) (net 1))
 (segment (start 158.58208 111.199999) (end 169.1 111.2) (width 0.4) (layer F.Cu) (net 1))
 (segment (start 169.1 111.2) (end 170 112.1) (width 0.4) (layer F.Cu) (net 1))
 (segment (start 158.502081 111.12) (end 158.58208 111.199999) (width 0.4) (layer F.Cu) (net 1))
 (segment (start 157.3 111.12) (end 158.502081 111.12) (width 0.4) (layer F.Cu) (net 1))
 (via (at 164 95.45) (size 1.3) (layers F.Cu B.Cu) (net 5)))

